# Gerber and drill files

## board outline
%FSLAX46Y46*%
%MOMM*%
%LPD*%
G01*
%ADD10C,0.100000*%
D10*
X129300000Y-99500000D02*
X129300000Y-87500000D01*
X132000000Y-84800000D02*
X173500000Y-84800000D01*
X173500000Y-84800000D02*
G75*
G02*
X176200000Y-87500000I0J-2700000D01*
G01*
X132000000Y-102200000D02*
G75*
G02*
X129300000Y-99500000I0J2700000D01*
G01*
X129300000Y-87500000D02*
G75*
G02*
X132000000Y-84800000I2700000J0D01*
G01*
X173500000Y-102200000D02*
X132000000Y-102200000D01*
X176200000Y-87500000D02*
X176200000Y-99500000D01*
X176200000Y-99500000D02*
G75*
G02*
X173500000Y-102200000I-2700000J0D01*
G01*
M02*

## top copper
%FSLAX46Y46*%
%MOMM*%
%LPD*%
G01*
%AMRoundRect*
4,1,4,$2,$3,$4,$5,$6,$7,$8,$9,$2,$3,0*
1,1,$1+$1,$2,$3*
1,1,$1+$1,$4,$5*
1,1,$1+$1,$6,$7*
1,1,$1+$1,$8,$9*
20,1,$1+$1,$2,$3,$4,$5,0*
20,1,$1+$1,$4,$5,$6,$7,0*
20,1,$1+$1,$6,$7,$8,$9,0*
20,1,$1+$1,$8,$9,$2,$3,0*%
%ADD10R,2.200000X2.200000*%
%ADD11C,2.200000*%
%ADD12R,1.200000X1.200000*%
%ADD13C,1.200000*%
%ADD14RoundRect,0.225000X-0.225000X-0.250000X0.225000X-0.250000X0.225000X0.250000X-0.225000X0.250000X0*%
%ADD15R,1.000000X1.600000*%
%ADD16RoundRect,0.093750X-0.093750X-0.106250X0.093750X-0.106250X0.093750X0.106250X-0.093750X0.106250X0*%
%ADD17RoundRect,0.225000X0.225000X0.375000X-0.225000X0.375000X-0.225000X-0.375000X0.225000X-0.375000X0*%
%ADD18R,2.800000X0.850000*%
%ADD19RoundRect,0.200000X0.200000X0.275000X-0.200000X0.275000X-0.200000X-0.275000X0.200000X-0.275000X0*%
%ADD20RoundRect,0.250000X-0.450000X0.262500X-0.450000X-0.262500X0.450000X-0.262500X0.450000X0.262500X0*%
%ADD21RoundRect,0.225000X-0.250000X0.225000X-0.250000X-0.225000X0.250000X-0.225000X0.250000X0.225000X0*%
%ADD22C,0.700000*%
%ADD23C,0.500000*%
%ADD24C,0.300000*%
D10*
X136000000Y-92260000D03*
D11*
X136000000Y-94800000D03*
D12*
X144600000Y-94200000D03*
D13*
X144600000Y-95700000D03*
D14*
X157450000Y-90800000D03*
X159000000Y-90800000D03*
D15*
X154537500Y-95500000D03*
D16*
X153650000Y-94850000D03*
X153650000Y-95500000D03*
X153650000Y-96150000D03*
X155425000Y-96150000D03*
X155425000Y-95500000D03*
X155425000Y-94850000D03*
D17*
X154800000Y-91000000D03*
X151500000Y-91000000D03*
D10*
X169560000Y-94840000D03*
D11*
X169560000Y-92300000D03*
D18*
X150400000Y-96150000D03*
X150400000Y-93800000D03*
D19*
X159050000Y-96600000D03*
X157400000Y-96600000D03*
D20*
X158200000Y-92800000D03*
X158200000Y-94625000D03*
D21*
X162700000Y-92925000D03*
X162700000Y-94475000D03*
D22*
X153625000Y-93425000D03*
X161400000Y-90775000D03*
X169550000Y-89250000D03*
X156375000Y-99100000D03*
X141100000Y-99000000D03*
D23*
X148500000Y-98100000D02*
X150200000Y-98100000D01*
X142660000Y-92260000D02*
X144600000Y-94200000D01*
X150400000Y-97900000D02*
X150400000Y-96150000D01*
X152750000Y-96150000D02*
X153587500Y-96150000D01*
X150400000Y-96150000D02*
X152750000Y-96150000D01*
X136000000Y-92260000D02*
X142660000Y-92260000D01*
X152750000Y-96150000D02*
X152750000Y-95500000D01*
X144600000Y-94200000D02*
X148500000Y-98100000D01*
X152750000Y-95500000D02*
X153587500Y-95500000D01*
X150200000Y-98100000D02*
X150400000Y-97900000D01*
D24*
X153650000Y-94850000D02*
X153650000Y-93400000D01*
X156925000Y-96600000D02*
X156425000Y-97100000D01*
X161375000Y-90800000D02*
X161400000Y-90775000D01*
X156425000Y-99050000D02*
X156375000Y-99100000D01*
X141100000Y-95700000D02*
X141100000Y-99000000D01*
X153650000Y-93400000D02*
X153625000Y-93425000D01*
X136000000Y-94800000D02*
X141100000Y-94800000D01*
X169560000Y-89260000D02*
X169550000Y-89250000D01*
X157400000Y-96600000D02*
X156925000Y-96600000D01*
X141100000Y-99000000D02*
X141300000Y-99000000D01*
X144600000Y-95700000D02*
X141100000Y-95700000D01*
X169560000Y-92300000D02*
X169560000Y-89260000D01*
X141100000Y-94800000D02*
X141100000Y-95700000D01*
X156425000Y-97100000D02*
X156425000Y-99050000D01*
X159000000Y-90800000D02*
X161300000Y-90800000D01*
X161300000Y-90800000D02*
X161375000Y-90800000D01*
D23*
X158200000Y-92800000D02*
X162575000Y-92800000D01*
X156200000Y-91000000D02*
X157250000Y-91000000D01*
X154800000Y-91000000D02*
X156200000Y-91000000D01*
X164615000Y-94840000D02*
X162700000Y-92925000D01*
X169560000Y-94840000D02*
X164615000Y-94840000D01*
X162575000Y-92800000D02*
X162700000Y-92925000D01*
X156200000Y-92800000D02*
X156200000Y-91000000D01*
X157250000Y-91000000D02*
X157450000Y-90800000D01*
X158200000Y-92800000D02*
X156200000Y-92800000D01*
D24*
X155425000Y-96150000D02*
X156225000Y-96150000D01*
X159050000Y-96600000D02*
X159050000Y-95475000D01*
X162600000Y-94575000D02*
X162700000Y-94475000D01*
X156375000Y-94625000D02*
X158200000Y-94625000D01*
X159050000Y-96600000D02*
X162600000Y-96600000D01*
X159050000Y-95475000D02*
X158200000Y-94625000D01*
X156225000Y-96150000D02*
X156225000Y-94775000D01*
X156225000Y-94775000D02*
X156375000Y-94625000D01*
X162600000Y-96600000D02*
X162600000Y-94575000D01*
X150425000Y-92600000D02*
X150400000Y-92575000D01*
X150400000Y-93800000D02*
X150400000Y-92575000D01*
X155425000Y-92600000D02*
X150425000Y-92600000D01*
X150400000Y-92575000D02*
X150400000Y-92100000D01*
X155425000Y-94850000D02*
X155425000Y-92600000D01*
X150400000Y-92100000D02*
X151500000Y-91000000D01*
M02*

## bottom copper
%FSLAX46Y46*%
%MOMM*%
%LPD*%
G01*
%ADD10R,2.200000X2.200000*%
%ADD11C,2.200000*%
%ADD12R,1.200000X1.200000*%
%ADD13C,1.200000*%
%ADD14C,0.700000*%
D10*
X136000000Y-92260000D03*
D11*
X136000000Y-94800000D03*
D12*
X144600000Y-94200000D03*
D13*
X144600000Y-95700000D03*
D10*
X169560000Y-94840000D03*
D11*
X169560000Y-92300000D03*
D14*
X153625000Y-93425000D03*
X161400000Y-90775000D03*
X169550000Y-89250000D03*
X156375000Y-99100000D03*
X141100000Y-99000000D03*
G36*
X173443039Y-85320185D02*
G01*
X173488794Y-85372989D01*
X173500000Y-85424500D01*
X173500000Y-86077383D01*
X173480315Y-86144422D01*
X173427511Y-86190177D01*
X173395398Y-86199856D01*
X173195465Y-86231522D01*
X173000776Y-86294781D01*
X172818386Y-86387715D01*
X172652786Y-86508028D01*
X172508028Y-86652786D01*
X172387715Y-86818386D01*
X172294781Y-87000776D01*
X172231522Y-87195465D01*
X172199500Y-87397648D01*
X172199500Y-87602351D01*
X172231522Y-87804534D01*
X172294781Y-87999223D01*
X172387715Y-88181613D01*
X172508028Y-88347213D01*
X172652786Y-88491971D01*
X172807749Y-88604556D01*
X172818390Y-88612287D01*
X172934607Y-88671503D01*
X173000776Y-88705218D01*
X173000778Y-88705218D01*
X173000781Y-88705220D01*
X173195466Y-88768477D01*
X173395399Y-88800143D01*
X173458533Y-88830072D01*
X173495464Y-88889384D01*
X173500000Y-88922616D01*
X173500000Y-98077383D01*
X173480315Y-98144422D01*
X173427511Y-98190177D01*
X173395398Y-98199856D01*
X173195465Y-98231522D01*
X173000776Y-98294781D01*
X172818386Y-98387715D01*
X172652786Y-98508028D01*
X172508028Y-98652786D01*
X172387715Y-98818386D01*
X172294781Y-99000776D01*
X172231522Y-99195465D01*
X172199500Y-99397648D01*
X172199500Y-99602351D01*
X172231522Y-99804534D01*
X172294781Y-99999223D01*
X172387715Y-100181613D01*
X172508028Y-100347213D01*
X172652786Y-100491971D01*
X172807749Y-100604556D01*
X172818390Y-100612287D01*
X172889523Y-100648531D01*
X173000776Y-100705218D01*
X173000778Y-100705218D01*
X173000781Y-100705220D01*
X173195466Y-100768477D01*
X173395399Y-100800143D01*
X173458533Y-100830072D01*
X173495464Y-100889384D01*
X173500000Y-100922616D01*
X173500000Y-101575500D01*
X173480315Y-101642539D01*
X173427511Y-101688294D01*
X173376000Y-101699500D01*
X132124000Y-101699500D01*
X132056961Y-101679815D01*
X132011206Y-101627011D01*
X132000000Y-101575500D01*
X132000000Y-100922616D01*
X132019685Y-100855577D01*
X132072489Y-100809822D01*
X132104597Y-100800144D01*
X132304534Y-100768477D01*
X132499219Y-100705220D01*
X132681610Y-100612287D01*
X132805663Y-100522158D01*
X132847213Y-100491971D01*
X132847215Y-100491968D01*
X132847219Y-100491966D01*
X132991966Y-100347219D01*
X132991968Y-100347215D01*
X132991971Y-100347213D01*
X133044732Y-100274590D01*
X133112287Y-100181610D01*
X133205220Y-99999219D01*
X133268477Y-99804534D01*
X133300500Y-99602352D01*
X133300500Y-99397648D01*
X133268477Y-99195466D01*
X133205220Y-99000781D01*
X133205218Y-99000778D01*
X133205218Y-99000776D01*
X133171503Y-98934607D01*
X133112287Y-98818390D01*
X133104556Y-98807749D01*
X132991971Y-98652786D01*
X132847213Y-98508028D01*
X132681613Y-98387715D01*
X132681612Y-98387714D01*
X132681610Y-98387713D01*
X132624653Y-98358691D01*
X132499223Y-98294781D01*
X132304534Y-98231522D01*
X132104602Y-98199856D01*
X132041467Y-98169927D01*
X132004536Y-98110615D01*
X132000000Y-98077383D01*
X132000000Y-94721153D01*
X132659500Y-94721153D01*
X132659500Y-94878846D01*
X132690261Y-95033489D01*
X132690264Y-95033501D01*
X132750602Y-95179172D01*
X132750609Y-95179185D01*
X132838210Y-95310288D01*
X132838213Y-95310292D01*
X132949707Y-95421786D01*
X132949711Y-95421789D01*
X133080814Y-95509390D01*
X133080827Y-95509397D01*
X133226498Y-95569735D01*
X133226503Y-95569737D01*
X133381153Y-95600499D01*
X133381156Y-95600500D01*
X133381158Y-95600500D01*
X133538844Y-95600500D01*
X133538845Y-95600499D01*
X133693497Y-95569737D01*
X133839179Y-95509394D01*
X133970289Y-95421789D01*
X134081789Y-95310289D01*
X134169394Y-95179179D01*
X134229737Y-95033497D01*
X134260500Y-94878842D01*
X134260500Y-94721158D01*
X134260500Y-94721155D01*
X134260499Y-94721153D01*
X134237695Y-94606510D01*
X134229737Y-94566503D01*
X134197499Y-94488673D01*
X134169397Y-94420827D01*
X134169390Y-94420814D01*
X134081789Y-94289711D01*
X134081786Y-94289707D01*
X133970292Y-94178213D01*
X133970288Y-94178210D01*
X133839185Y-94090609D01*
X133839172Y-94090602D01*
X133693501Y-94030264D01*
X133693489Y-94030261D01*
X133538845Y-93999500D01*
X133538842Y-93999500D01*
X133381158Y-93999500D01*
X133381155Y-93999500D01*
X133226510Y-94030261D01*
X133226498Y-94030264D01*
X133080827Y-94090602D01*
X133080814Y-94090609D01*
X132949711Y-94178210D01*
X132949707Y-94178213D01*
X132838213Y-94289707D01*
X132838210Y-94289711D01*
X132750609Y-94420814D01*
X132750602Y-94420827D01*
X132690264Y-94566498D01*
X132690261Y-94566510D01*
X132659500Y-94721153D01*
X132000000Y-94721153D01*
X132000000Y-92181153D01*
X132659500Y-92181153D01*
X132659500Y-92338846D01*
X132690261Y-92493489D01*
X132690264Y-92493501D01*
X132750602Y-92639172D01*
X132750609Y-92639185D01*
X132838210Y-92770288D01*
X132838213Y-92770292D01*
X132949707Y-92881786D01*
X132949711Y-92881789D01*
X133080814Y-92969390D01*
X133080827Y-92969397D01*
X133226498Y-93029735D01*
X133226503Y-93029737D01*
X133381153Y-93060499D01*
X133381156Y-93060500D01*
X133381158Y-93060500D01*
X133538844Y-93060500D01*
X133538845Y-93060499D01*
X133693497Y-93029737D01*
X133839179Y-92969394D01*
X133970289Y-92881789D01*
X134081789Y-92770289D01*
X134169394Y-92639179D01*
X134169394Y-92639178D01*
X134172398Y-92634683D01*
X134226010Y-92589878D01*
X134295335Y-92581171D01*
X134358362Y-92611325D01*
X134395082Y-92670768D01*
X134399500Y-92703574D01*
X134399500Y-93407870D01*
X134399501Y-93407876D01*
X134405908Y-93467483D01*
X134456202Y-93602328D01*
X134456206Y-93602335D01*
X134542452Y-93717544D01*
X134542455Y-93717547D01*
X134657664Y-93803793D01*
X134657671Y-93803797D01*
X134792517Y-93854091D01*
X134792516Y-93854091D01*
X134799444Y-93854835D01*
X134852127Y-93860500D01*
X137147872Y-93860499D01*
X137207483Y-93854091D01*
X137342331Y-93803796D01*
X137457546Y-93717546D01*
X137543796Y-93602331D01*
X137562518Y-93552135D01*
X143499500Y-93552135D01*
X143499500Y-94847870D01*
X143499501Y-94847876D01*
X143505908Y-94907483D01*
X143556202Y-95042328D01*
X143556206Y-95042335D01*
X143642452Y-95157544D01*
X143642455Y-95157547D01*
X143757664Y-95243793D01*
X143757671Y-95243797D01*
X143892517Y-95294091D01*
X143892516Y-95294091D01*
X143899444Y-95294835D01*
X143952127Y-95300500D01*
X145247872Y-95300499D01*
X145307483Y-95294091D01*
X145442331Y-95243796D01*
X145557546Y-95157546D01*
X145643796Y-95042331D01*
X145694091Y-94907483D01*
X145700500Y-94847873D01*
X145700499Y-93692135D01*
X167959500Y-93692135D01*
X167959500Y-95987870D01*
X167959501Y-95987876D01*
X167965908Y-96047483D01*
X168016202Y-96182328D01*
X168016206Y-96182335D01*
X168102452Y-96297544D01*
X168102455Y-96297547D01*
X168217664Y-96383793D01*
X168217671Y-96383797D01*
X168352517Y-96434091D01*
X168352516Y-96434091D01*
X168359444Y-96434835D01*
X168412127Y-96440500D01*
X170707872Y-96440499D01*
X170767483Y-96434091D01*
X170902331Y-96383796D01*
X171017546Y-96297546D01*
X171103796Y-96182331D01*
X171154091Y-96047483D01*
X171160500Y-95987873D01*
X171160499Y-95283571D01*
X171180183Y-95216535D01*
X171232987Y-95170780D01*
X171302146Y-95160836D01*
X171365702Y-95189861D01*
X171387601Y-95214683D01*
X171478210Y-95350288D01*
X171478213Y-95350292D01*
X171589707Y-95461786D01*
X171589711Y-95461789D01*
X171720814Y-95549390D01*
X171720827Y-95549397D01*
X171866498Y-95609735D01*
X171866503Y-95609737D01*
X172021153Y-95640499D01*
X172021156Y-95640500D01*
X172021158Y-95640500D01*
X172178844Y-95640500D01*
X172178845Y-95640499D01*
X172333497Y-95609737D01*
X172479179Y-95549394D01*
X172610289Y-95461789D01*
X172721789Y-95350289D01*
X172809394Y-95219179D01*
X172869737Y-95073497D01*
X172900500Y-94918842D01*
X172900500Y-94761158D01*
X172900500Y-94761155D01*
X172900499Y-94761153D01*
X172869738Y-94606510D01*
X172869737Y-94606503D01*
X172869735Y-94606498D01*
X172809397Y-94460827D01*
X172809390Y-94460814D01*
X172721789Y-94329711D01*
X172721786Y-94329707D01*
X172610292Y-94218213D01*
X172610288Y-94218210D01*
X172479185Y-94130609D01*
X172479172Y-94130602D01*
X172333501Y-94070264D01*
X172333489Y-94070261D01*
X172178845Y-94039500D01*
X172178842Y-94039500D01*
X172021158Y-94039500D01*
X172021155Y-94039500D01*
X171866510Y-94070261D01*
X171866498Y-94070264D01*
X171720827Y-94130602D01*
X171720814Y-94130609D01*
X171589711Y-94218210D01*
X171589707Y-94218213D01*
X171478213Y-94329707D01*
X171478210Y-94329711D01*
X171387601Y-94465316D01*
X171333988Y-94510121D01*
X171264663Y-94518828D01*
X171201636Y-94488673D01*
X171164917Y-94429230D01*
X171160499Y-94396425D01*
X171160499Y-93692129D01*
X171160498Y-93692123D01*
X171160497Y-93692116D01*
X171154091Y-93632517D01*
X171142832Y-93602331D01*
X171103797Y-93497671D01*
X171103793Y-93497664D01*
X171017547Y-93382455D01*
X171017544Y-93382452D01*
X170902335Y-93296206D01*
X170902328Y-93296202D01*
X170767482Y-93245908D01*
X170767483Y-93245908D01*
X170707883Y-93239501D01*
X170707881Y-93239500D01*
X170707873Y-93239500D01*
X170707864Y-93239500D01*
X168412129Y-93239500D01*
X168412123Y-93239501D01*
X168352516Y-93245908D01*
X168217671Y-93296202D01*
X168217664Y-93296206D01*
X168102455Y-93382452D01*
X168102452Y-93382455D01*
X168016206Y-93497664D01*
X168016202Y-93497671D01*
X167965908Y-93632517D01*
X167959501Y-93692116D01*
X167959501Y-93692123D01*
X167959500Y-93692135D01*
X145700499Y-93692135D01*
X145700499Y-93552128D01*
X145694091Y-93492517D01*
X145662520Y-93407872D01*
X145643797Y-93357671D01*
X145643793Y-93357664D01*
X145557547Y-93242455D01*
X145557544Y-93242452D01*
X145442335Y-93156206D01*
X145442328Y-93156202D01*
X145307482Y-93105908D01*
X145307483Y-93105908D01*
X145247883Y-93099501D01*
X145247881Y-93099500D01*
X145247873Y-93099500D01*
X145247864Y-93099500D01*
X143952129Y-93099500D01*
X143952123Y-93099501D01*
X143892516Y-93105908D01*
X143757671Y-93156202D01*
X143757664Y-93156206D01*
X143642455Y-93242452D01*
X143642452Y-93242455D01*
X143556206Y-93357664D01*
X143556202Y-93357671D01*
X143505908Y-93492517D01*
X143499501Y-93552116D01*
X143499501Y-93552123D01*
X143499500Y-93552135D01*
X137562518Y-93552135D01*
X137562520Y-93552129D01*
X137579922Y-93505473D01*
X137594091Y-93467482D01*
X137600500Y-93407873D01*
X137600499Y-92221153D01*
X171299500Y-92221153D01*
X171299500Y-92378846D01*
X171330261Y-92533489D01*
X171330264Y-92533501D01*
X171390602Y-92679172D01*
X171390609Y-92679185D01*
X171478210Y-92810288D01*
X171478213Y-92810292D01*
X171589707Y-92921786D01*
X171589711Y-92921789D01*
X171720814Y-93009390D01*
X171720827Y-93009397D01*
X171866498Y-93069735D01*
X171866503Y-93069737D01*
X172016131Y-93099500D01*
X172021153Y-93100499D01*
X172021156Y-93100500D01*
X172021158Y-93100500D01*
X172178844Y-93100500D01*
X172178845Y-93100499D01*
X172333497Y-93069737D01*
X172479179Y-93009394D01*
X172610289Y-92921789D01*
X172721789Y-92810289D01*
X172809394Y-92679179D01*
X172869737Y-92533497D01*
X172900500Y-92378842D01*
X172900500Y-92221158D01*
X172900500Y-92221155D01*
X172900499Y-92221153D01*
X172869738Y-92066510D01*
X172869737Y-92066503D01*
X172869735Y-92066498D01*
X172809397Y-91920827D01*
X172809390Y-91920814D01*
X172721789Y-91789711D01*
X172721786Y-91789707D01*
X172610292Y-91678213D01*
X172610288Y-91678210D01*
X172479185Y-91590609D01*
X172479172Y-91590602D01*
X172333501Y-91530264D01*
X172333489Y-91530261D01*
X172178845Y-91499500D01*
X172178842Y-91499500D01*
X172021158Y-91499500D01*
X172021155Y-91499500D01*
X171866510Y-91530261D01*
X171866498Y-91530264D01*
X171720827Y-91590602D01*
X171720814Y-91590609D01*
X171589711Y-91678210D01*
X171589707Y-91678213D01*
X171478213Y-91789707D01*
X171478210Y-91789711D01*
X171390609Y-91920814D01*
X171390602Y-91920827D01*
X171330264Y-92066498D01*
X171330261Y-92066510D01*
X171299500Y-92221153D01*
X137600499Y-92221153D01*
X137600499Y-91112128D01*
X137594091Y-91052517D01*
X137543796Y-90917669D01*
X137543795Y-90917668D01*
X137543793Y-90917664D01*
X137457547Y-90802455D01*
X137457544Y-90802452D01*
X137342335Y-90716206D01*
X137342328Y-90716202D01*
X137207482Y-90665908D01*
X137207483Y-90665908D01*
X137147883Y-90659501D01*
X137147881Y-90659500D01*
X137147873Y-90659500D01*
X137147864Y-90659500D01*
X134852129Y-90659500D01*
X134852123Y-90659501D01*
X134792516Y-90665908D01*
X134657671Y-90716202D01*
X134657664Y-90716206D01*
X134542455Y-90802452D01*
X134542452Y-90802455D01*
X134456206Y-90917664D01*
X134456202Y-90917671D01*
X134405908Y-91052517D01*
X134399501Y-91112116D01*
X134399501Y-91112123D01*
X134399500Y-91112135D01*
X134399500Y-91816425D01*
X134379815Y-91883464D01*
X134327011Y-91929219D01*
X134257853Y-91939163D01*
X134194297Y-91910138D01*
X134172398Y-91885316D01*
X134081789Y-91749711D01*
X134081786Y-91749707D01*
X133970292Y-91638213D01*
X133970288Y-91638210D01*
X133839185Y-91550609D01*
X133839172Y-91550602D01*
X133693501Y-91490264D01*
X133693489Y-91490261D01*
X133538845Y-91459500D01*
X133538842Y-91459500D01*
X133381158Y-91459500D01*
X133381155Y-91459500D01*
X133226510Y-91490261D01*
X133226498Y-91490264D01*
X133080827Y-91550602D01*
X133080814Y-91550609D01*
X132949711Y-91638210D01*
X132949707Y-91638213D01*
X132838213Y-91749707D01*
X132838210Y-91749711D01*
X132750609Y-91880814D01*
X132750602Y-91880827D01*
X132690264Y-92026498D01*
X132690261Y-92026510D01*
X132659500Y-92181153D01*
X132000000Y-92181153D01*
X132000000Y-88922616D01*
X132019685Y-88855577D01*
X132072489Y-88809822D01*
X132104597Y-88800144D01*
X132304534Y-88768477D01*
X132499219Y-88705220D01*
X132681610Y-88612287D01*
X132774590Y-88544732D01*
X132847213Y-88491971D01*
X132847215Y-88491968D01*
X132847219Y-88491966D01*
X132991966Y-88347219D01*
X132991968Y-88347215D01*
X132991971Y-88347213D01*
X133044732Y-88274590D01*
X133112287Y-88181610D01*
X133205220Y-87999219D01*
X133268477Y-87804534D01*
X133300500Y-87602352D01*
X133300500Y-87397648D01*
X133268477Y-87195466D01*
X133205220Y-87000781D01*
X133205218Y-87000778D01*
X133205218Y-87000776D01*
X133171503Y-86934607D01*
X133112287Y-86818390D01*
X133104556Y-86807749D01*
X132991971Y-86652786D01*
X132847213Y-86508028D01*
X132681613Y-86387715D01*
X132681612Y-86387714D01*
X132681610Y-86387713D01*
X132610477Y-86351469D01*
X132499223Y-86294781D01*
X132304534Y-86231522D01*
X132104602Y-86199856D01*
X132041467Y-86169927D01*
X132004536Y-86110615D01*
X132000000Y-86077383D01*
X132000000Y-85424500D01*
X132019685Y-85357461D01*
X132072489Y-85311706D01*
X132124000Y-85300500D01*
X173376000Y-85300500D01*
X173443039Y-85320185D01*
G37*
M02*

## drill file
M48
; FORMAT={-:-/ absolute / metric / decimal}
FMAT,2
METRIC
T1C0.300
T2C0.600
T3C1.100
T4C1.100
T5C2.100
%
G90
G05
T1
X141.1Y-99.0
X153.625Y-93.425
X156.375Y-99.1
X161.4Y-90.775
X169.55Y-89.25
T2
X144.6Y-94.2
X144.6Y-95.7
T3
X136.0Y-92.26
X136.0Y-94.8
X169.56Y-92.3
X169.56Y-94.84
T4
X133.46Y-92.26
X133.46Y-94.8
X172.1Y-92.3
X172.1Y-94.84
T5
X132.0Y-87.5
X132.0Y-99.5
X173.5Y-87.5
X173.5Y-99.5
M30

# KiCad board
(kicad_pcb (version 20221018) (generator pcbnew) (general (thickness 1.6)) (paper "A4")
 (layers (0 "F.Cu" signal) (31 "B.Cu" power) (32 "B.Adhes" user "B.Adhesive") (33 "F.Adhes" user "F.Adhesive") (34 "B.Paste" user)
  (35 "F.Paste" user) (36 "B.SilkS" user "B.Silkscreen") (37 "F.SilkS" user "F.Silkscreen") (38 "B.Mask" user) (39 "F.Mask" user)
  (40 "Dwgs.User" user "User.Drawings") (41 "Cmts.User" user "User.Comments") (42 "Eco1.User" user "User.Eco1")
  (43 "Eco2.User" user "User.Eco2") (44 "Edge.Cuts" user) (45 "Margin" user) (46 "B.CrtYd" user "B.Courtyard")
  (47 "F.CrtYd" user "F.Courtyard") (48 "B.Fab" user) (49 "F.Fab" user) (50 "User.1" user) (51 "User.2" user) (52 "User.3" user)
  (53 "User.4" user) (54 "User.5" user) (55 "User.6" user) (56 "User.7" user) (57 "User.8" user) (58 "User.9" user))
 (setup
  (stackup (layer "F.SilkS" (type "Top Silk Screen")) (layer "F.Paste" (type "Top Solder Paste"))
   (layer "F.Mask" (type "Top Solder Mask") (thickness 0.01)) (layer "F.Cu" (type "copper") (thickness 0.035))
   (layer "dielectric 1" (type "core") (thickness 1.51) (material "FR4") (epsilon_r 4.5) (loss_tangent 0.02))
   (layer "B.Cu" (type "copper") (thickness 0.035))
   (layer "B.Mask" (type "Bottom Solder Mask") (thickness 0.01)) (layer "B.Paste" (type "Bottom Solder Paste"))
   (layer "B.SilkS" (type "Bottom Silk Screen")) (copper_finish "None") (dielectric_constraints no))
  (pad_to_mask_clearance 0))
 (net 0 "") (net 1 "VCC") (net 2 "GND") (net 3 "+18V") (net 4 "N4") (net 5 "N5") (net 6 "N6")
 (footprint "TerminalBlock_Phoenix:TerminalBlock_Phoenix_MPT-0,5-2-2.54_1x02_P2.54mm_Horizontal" (layer "F.Cu") (at 136 92.26 -90)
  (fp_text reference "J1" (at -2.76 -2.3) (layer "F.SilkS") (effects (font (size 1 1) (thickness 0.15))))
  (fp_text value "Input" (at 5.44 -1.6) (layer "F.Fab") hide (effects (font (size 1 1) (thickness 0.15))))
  (pad "" np_thru_hole circle (at 0 2.54 270) (size 1.1 1.1) (drill 1.1) (layers "*.Cu" "*.Mask"))
  (pad "" np_thru_hole circle (at 2.54 2.54 270) (size 1.1 1.1) (drill 1.1) (layers "*.Cu" "*.Mask"))
  (pad "1" thru_hole rect (at 0 0 270) (size 2.2 2.2) (drill 1.1) (layers "*.Cu" "*.Mask") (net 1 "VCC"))
  (pad "2" thru_hole circle (at 2.54 0 270) (size 2.2 2.2) (drill 1.1) (layers "*.Cu" "*.Mask") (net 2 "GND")))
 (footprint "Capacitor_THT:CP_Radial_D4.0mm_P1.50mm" (layer "F.Cu") (at 144.6 94.2 -90)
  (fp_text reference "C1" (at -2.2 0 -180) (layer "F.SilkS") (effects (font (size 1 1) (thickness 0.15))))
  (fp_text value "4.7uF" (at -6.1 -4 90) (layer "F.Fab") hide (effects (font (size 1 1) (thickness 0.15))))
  (pad "1" thru_hole rect (at 0 0 270) (size 1.2 1.2) (drill 0.6) (layers "*.Cu" "*.Mask") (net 1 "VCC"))
  (pad "2" thru_hole circle (at 1.5 0 270) (size 1.2 1.2) (drill 0.6) (layers "*.Cu" "*.Mask") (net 2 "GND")))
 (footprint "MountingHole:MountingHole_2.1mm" (layer "F.Cu") (at 173.5 99.5)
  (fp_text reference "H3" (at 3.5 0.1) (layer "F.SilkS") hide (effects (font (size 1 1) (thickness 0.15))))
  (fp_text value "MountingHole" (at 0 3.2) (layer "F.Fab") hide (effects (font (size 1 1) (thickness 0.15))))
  (pad "" np_thru_hole circle (at 0 0) (size 2.1 2.1) (drill 2.1) (layers "*.Cu" "*.Mask")))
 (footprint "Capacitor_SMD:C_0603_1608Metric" (layer "F.Cu") (at 158.225 90.8)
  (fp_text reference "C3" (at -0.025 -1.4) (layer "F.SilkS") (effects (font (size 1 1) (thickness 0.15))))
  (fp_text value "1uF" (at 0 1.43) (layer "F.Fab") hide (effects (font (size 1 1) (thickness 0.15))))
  (pad "1" smd roundrect (at -0.775 0) (size 0.9 0.95) (layers "F.Cu" "F.Paste" "F.Mask") (roundrect_rratio 0.25) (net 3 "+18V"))
  (pad "2" smd roundrect (at 0.775 0) (size 0.9 0.95) (layers "F.Cu" "F.Paste" "F.Mask") (roundrect_rratio 0.25) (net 2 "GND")))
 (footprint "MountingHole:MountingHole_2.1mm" (layer "F.Cu") (at 173.5 87.5)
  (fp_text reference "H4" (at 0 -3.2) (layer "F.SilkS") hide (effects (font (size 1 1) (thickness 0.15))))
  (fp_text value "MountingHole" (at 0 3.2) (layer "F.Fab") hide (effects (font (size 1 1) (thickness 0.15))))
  (pad "" np_thru_hole circle (at 0 0) (size 2.1 2.1) (drill 2.1) (layers "*.Cu" "*.Mask")))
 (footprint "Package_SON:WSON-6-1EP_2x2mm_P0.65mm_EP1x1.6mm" (layer "F.Cu") (at 154.5375 95.5)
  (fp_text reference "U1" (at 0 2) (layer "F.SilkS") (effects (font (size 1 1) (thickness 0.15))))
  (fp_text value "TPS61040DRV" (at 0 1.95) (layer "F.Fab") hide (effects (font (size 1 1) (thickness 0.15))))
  (pad "" smd roundrect (at 0 -0.4) (size 0.81 0.64) (layers "F.Paste") (roundrect_rratio 0.25))
  (pad "" smd rect (at 0 0) (size 1 1.6) (layers "F.Cu"))
  (pad "" smd roundrect (at 0 0.4) (size 0.81 0.64) (layers "F.Paste") (roundrect_rratio 0.25))
  (pad "1" smd roundrect (at -0.8875 -0.65) (size 0.375 0.4) (layers "F.Cu" "F.Paste" "F.Mask") (roundrect_rratio 0.25) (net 2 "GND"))
  (pad "2" smd roundrect (at -0.8875 0) (size 0.375 0.4) (layers "F.Cu" "F.Paste" "F.Mask") (roundrect_rratio 0.25) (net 1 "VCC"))
  (pad "3" smd roundrect (at -0.8875 0.65) (size 0.375 0.4) (layers "F.Cu" "F.Paste" "F.Mask") (roundrect_rratio 0.25) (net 1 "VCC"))
  (pad "4" smd roundrect (at 0.8875 0.65) (size 0.375 0.4) (layers "F.Cu" "F.Paste" "F.Mask") (roundrect_rratio 0.25) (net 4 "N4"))
  (pad "5" smd roundrect (at 0.8875 0) (size 0.375 0.4) (layers "F.Cu" "F.Paste" "F.Mask") (roundrect_rratio 0.25) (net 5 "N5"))
  (pad "6" smd roundrect (at 0.8875 -0.65) (size 0.375 0.4) (layers "F.Cu" "F.Paste" "F.Mask") (roundrect_rratio 0.25) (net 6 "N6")))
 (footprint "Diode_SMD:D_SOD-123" (layer "F.Cu") (at 153.15 91 180)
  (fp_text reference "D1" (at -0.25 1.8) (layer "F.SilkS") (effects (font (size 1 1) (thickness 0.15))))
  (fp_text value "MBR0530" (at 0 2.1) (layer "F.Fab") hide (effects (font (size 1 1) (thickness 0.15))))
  (pad "1" smd roundrect (at -1.65 0 180) (size 0.9 1.2) (layers "F.Cu" "F.Paste" "F.Mask") (roundrect_rratio 0.25) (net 3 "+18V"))
  (pad "2" smd roundrect (at 1.65 0 180) (size 0.9 1.2) (layers "F.Cu" "F.Paste" "F.Mask") (roundrect_rratio 0.25) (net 6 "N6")))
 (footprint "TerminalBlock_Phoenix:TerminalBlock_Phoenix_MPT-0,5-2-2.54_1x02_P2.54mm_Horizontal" (layer "F.Cu") (at 169.56 94.84 90)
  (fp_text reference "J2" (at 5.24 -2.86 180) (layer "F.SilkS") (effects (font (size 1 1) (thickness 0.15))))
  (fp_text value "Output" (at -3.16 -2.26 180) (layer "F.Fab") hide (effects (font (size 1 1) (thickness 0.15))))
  (pad "" np_thru_hole circle (at 0 2.54 90) (size 1.1 1.1) (drill 1.1) (layers "*.Cu" "*.Mask"))
  (pad "" np_thru_hole circle (at 2.54 2.54 90) (size 1.1 1.1) (drill 1.1) (layers "*.Cu" "*.Mask"))
  (pad "1" thru_hole rect (at 0 0 90) (size 2.2 2.2) (drill 1.1) (layers "*.Cu" "*.Mask") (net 3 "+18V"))
  (pad "2" thru_hole circle (at 2.54 0 90) (size 2.2 2.2) (drill 1.1) (layers "*.Cu" "*.Mask") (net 2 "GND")))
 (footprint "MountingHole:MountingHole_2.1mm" (layer "F.Cu") (at 132 87.5)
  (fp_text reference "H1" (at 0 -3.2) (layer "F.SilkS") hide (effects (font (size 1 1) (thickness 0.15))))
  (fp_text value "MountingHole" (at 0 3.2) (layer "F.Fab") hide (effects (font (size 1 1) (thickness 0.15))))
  (pad "" np_thru_hole circle (at 0 0) (size 2.1 2.1) (drill 2.1) (layers "*.Cu" "*.Mask")))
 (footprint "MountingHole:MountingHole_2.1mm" (layer "F.Cu") (at 132 99.5)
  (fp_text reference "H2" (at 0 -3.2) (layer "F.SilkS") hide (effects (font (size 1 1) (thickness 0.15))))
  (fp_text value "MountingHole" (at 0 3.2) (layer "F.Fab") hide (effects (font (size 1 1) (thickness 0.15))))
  (pad "" np_thru_hole circle (at 0 0) (size 2.1 2.1) (drill 2.1) (layers "*.Cu" "*.Mask")))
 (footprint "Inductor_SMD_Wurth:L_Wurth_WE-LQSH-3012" (layer "F.Cu") (at 150.4 94.975 90)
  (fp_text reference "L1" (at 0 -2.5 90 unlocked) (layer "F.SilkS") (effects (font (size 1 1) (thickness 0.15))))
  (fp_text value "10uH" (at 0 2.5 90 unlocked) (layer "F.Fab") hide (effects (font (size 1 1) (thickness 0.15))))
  (pad "1" smd rect (at -1.175 0 90) (size 0.85 2.8) (layers "F.Cu" "F.Paste" "F.Mask") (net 1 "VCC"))
  (pad "2" smd rect (at 1.175 0 90) (size 0.85 2.8) (layers "F.Cu" "F.Paste" "F.Mask") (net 6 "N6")))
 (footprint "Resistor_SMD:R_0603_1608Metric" (layer "F.Cu") (at 158.225 96.6 180)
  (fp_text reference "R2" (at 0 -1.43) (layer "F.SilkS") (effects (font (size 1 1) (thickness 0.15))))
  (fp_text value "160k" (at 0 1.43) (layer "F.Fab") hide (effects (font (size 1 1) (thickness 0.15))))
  (pad "1" smd roundrect (at -0.825 0 180) (size 0.8 0.95) (layers "F.Cu" "F.Paste" "F.Mask") (roundrect_rratio 0.25) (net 4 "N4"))
  (pad "2" smd roundrect (at 0.825 0 180) (size 0.8 0.95) (layers "F.Cu" "F.Paste" "F.Mask") (roundrect_rratio 0.25) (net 2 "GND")))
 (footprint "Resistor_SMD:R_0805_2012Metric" (layer "F.Cu") (at 158.2 93.7125 -90)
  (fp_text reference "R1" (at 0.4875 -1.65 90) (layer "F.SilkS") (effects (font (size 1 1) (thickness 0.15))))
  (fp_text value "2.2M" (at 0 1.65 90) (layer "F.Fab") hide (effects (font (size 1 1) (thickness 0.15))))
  (pad "1" smd roundrect (at -0.9125 0 270) (size 1.025 1.4) (layers "F.Cu" "F.Paste" "F.Mask") (roundrect_rratio 0.243902) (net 3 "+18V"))
  (pad "2" smd roundrect (at 0.9125 0 270) (size 1.025 1.4) (layers "F.Cu" "F.Paste" "F.Mask") (roundrect_rratio 0.243902) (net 4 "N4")))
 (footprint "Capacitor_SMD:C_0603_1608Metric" (layer "F.Cu") (at 162.7 93.7 -90)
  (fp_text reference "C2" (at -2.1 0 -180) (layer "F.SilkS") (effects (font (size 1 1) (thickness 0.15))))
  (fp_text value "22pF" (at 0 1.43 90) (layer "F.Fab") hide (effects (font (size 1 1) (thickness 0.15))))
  (pad "1" smd roundrect (at -0.775 0 270) (size 0.9 0.95) (layers "F.Cu" "F.Paste" "F.Mask") (roundrect_rratio 0.25) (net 3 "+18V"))
  (pad "2" smd roundrect (at 0.775 0 270) (size 0.9 0.95) (layers "F.Cu" "F.Paste" "F.Mask") (roundrect_rratio 0.25) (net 4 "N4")))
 (gr_line (start 129.3 99.5) (end 129.3 87.5) (stroke (width 0.1) (type default)) (layer "Edge.Cuts"))
 (gr_line (start 132 84.8) (end 173.5 84.8) (stroke (width 0.1) (type default)) (layer "Edge.Cuts"))
 (gr_arc (start 173.5 84.8) (mid 175.409188 85.590812) (end 176.2 87.5) (stroke (width 0.1) (type default)) (layer "Edge.Cuts"))
 (gr_arc (start 132 102.2) (mid 130.090812 101.409188) (end 129.3 99.5) (stroke (width 0.1) (type default)) (layer "Edge.Cuts"))
 (gr_arc (start 129.3 87.5) (mid 130.090812 85.590812) (end 132 84.8) (stroke (width 0.1) (type default)) (layer "Edge.Cuts"))
 (gr_line (start 173.5 102.2) (end 132 102.2) (stroke (width 0.1) (type default)) (layer "Edge.Cuts"))
 (gr_line (start 176.2 87.5) (end 176.2 99.5) (stroke (width 0.1) (type default)) (layer "Edge.Cuts"))
 (gr_arc (start 176.2 99.5) (mid 175.409188 101.409188) (end 173.5 102.2) (stroke (width 0.1) (type default)) (layer "Edge.Cuts"))
 (segment (start 148.5 98.1) (end 150.2 98.1) (width 0.5) (layer "F.Cu") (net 1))
 (segment (start 142.66 92.26) (end 144.6 94.2) (width 0.5) (layer "F.Cu") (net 1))
 (segment (start 150.4 97.9) (end 150.4 96.15) (width 0.5) (layer "F.Cu") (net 1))
 (segment (start 152.75 96.15) (end 153.5875 96.15) (width 0.5) (layer "F.Cu") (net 1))
 (segment (start 150.4 96.15) (end 152.75 96.15) (width 0.5) (layer "F.Cu") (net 1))
 (segment (start 136 92.26) (end 142.66 92.26) (width 0.5) (layer "F.Cu") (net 1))
 (segment (start 152.75 96.15) (end 152.75 95.5) (width 0.5) (layer "F.Cu") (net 1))
 (segment (start 144.6 94.2) (end 148.5 98.1) (width 0.5) (layer "F.Cu") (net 1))
 (segment (start 152.75 95.5) (end 153.5875 95.5) (width 0.5) (layer "F.Cu") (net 1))
 (segment (start 150.2 98.1) (end 150.4 97.9) (width 0.5) (layer "F.Cu") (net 1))
 (segment (start 153.65 94.85) (end 153.65 93.4) (width 0.3) (layer "F.Cu") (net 2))
 (segment (start 156.925 96.6) (end 156.425 97.1) (width 0.3) (layer "F.Cu") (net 2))
 (segment (start 161.375 90.8) (end 161.4 90.775) (width 0.3) (layer "F.Cu") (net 2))
 (segment (start 156.425 99.05) (end 156.375 99.1) (width 0.3) (layer "F.Cu") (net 2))
 (segment (start 141.1 95.7) (end 141.1 99) (width 0.3) (layer "F.Cu") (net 2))
 (segment (start 153.65 93.4) (end 153.625 93.425) (width 0.3) (layer "F.Cu") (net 2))
 (segment (start 136 94.8) (end 141.1 94.8) (width 0.3) (layer "F.Cu") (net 2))
 (segment (start 169.56 89.26) (end 169.55 89.25) (width 0.3) (layer "F.Cu") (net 2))
 (segment (start 157.4 96.6) (end 156.925 96.6) (width 0.3) (layer "F.Cu") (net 2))
 (segment (start 141.1 99) (end 141.3 99) (width 0.3) (layer "F.Cu") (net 2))
 (segment (start 144.6 95.7) (end 141.1 95.7) (width 0.3) (layer "F.Cu") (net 2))
 (segment (start 169.56 92.3) (end 169.56 89.26) (width 0.3) (layer "F.Cu") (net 2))
 (segment (start 141.1 94.8) (end 141.1 95.7) (width 0.3) (layer "F.Cu") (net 2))
 (segment (start 156.425 97.1) (end 156.425 99.05) (width 0.3) (layer "F.Cu") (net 2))
 (segment (start 159 90.8) (end 161.3 90.8) (width 0.3) (layer "F.Cu") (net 2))
 (segment (start 161.3 90.8) (end 161.375 90.8) (width 0.3) (layer "F.Cu") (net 2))
 (via (at 153.625 93.425) (size 0.7) (drill 0.3) (layers "F.Cu" "B.Cu") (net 2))
 (via (at 161.4 90.775) (size 0.7) (drill 0.3) (layers "F.Cu" "B.Cu") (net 2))
 (via (at 169.55 89.25) (size 0.7) (drill 0.3) (layers "F.Cu" "B.Cu") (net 2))
 (via (at 156.375 99.1) (size 0.7) (drill 0.3) (layers "F.Cu" "B.Cu") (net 2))
 (via (at 141.1 99) (size 0.7) (drill 0.3) (layers "F.Cu" "B.Cu") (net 2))
 (segment (start 158.2 92.8) (end 162.575 92.8) (width 0.5) (layer "F.Cu") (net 3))
 (segment (start 156.2 91) (end 157.25 91) (width 0.5) (layer "F.Cu") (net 3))
 (segment (start 154.8 91) (end 156.2 91) (width 0.5) (layer "F.Cu") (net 3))
 (segment (start 164.615 94.84) (end 162.7 92.925) (width 0.5) (layer "F.Cu") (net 3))
 (segment (start 169.56 94.84) (end 164.615 94.84) (width 0.5) (layer "F.Cu") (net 3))
 (segment (start 162.575 92.8) (end 162.7 92.925) (width 0.5) (layer "F.Cu") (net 3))
 (segment (start 156.2 92.8) (end 156.2 91) (width 0.5) (layer "F.Cu") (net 3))
 (segment (start 157.25 91) (end 157.45 90.8) (width 0.5) (layer "F.Cu") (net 3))
 (segment (start 158.2 92.8) (end 156.2 92.8) (width 0.5) (layer "F.Cu") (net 3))
 (segment (start 155.425 96.15) (end 156.225 96.15) (width 0.3) (layer "F.Cu") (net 4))
 (segment (start 159.05 96.6) (end 159.05 95.475) (width 0.3) (layer "F.Cu") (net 4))
 (segment (start 162.6 94.575) (end 162.7 94.475) (width 0.3) (layer "F.Cu") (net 4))
 (segment (start 156.375 94.625) (end 158.2 94.625) (width 0.3) (layer "F.Cu") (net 4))
 (segment (start 159.05 96.6) (end 162.6 96.6) (width 0.3) (layer "F.Cu") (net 4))
 (segment (start 159.05 95.475) (end 158.2 94.625) (width 0.3) (layer "F.Cu") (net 4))
 (segment (start 156.225 96.15) (end 156.225 94.775) (width 0.3) (layer "F.Cu") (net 4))
 (segment (start 156.225 94.775) (end 156.375 94.625) (width 0.3) (layer "F.Cu") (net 4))
 (segment (start 162.6 96.6) (end 162.6 94.575) (width 0.3) (layer "F.Cu") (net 4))
 (segment (start 150.425 92.6) (end 150.4 92.575) (width 0.3) (layer "F.Cu") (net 6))
 (segment (start 150.4 93.8) (end 150.4 92.575) (width 0.3) (layer "F.Cu") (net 6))
 (segment (start 155.425 92.6) (end 150.425 92.6) (width 0.3) (layer "F.Cu") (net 6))
 (segment (start 150.4 92.575) (end 150.4 92.1) (width 0.3) (layer "F.Cu") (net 6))
 (segment (start 155.425 94.85) (end 155.425 92.6) (width 0.3) (layer "F.Cu") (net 6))
 (segment (start 150.4 92.1) (end 151.5 91) (width 0.3) (layer "F.Cu") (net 6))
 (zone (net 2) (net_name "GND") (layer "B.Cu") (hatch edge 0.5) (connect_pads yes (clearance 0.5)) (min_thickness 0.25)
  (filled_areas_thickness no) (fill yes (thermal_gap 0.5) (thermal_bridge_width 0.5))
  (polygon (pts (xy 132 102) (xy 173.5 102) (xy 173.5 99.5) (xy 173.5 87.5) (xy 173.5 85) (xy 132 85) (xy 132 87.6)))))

